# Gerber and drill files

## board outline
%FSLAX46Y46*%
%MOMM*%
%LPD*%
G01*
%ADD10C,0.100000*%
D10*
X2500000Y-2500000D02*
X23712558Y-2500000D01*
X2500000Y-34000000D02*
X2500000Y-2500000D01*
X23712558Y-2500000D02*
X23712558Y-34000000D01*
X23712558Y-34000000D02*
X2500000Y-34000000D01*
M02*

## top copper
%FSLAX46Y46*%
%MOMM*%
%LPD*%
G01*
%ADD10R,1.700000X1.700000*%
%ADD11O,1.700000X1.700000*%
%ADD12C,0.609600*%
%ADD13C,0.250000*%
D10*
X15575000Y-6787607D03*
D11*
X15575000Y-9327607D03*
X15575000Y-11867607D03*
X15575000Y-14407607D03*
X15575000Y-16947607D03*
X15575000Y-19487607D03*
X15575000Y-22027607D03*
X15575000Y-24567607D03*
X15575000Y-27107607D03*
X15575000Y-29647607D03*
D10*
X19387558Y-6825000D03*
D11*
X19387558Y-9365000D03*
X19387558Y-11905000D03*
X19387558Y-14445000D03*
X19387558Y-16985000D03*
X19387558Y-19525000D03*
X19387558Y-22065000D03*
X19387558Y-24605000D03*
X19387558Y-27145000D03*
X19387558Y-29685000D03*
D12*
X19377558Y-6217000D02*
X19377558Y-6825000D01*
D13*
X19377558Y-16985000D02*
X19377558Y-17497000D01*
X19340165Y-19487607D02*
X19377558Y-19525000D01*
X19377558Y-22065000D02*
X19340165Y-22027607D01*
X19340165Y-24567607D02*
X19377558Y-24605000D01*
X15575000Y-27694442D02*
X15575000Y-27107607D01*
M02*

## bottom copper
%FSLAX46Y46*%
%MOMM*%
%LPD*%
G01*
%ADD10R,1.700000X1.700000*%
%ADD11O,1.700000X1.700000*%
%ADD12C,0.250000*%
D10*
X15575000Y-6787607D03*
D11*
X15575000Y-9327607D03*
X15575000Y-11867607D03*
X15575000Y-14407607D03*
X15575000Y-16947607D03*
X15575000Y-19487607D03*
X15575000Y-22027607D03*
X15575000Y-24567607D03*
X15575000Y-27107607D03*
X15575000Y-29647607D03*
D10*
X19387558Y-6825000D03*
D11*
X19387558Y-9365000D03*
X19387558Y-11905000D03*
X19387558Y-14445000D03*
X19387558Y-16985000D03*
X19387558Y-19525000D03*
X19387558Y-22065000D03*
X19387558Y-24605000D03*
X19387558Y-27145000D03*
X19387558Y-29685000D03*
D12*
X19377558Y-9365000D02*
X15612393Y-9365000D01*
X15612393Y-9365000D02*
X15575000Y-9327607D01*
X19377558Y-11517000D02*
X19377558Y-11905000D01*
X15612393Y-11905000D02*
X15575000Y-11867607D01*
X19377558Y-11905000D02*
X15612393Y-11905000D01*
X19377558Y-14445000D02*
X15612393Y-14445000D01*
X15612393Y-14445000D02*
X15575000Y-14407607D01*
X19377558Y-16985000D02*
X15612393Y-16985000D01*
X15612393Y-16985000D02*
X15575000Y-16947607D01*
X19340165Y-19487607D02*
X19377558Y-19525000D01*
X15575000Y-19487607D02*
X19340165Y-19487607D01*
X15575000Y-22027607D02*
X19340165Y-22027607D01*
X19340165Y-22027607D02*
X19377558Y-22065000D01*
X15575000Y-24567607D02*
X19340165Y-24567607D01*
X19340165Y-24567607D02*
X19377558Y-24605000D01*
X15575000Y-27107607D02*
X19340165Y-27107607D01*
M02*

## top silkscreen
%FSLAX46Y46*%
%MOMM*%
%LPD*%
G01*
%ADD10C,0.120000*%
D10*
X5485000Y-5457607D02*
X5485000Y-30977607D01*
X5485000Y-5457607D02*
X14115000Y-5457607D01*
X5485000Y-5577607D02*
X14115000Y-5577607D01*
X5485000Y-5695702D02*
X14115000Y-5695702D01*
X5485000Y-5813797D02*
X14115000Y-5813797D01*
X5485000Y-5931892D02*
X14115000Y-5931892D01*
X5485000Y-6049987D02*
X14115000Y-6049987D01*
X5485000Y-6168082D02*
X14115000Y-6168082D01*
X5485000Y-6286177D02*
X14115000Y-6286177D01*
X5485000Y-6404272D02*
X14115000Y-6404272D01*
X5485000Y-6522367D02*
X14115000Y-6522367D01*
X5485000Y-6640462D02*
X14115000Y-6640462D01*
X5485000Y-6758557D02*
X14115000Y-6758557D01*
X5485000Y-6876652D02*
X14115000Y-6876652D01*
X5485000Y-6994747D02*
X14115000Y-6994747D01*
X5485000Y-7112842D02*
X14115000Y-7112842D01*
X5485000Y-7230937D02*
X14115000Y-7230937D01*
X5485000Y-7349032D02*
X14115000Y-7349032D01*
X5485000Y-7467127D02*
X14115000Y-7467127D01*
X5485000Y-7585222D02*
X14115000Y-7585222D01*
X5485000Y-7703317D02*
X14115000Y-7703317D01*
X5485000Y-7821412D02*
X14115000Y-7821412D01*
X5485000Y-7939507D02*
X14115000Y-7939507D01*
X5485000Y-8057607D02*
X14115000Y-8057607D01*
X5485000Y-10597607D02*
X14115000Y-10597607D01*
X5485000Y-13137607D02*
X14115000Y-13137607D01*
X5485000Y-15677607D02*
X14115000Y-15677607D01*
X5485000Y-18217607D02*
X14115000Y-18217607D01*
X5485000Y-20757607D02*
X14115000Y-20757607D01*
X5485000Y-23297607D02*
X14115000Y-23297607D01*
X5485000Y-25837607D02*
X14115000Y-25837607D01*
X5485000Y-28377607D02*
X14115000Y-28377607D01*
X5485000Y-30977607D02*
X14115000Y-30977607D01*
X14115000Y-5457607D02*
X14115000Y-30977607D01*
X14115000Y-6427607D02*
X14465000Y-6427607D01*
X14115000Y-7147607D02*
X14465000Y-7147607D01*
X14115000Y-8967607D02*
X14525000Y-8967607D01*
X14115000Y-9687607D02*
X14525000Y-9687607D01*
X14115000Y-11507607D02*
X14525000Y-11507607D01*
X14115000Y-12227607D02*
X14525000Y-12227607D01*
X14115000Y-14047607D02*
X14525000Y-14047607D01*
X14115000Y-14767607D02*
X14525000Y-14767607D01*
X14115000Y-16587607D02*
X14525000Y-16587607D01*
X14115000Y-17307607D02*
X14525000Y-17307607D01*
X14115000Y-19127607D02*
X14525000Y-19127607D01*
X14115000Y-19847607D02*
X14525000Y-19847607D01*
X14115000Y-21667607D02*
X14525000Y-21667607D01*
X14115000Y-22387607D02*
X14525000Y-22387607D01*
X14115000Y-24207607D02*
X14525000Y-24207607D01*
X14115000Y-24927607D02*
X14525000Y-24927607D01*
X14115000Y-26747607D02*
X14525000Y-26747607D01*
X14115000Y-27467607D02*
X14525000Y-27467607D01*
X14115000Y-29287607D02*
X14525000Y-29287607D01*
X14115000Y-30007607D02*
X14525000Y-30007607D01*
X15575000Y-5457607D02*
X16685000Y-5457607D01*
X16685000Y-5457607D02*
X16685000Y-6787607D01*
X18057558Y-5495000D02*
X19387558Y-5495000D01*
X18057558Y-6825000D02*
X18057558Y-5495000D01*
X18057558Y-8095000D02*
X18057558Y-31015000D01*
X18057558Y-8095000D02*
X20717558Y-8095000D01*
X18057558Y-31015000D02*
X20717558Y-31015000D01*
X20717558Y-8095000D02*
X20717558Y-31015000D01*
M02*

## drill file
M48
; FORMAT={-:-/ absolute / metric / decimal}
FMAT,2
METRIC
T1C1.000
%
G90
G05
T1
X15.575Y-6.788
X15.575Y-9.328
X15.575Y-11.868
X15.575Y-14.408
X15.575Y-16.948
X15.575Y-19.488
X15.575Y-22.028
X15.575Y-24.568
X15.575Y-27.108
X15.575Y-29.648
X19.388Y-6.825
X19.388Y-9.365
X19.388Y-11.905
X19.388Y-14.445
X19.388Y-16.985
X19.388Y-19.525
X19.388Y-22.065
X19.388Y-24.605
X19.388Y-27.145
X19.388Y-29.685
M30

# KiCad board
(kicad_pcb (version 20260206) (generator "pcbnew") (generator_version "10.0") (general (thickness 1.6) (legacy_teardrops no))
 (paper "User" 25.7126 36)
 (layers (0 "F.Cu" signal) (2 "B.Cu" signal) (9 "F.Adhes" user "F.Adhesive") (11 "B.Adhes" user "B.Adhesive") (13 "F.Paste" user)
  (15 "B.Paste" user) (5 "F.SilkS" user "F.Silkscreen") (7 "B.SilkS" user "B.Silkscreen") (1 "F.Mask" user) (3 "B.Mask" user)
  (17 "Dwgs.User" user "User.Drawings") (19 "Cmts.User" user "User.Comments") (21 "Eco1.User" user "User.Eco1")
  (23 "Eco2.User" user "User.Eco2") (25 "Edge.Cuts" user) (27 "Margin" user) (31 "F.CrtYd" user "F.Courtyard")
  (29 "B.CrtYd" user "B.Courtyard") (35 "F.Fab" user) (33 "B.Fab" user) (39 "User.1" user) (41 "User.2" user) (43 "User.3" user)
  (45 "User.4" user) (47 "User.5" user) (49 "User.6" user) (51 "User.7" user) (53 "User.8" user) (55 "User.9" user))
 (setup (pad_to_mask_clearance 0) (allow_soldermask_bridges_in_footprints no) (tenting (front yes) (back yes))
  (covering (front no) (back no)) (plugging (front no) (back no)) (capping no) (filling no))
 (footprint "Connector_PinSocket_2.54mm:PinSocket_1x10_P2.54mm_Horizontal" (layer "F.Cu") (at 15.575 6.787607)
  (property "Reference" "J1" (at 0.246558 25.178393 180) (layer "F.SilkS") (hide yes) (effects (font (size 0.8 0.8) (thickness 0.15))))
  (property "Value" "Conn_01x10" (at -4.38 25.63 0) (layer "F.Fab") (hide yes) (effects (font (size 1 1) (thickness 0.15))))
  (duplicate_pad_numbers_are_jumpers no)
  (fp_line (start -10.09 -1.33) (end -10.09 24.19) (stroke (width 0.12) (type solid)) (layer "F.SilkS"))
  (fp_line (start -10.09 -1.33) (end -1.46 -1.33) (stroke (width 0.12) (type solid)) (layer "F.SilkS"))
  (fp_line (start -10.09 -1.21) (end -1.46 -1.21) (stroke (width 0.12) (type solid)) (layer "F.SilkS"))
  (fp_line (start -10.09 -1.091905) (end -1.46 -1.091905) (stroke (width 0.12) (type solid)) (layer "F.SilkS"))
  (fp_line (start -10.09 -0.97381) (end -1.46 -0.97381) (stroke (width 0.12) (type solid)) (layer "F.SilkS"))
  (fp_line (start -10.09 -0.855715) (end -1.46 -0.855715) (stroke (width 0.12) (type solid)) (layer "F.SilkS"))
  (fp_line (start -10.09 -0.73762) (end -1.46 -0.73762) (stroke (width 0.12) (type solid)) (layer "F.SilkS"))
  (fp_line (start -10.09 -0.619525) (end -1.46 -0.619525) (stroke (width 0.12) (type solid)) (layer "F.SilkS"))
  (fp_line (start -10.09 -0.50143) (end -1.46 -0.50143) (stroke (width 0.12) (type solid)) (layer "F.SilkS"))
  (fp_line (start -10.09 -0.383335) (end -1.46 -0.383335) (stroke (width 0.12) (type solid)) (layer "F.SilkS"))
  (fp_line (start -10.09 -0.26524) (end -1.46 -0.26524) (stroke (width 0.12) (type solid)) (layer "F.SilkS"))
  (fp_line (start -10.09 -0.147145) (end -1.46 -0.147145) (stroke (width 0.12) (type solid)) (layer "F.SilkS"))
  (fp_line (start -10.09 -0.02905) (end -1.46 -0.02905) (stroke (width 0.12) (type solid)) (layer "F.SilkS"))
  (fp_line (start -10.09 0.089045) (end -1.46 0.089045) (stroke (width 0.12) (type solid)) (layer "F.SilkS"))
  (fp_line (start -10.09 0.20714) (end -1.46 0.20714) (stroke (width 0.12) (type solid)) (layer "F.SilkS"))
  (fp_line (start -10.09 0.325235) (end -1.46 0.325235) (stroke (width 0.12) (type solid)) (layer "F.SilkS"))
  (fp_line (start -10.09 0.44333) (end -1.46 0.44333) (stroke (width 0.12) (type solid)) (layer "F.SilkS"))
  (fp_line (start -10.09 0.561425) (end -1.46 0.561425) (stroke (width 0.12) (type solid)) (layer "F.SilkS"))
  (fp_line (start -10.09 0.67952) (end -1.46 0.67952) (stroke (width 0.12) (type solid)) (layer "F.SilkS"))
  (fp_line (start -10.09 0.797615) (end -1.46 0.797615) (stroke (width 0.12) (type solid)) (layer "F.SilkS"))
  (fp_line (start -10.09 0.91571) (end -1.46 0.91571) (stroke (width 0.12) (type solid)) (layer "F.SilkS"))
  (fp_line (start -10.09 1.033805) (end -1.46 1.033805) (stroke (width 0.12) (type solid)) (layer "F.SilkS"))
  (fp_line (start -10.09 1.1519) (end -1.46 1.1519) (stroke (width 0.12) (type solid)) (layer "F.SilkS"))
  (fp_line (start -10.09 1.27) (end -1.46 1.27) (stroke (width 0.12) (type solid)) (layer "F.SilkS"))
  (fp_line (start -10.09 3.81) (end -1.46 3.81) (stroke (width 0.12) (type solid)) (layer "F.SilkS"))
  (fp_line (start -10.09 6.35) (end -1.46 6.35) (stroke (width 0.12) (type solid)) (layer "F.SilkS"))
  (fp_line (start -10.09 8.89) (end -1.46 8.89) (stroke (width 0.12) (type solid)) (layer "F.SilkS"))
  (fp_line (start -10.09 11.43) (end -1.46 11.43) (stroke (width 0.12) (type solid)) (layer "F.SilkS"))
  (fp_line (start -10.09 13.97) (end -1.46 13.97) (stroke (width 0.12) (type solid)) (layer "F.SilkS"))
  (fp_line (start -10.09 16.51) (end -1.46 16.51) (stroke (width 0.12) (type solid)) (layer "F.SilkS"))
  (fp_line (start -10.09 19.05) (end -1.46 19.05) (stroke (width 0.12) (type solid)) (layer "F.SilkS"))
  (fp_line (start -10.09 21.59) (end -1.46 21.59) (stroke (width 0.12) (type solid)) (layer "F.SilkS"))
  (fp_line (start -10.09 24.19) (end -1.46 24.19) (stroke (width 0.12) (type solid)) (layer "F.SilkS"))
  (fp_line (start -1.46 -1.33) (end -1.46 24.19) (stroke (width 0.12) (type solid)) (layer "F.SilkS"))
  (fp_line (start -1.46 -0.36) (end -1.11 -0.36) (stroke (width 0.12) (type solid)) (layer "F.SilkS"))
  (fp_line (start -1.46 0.36) (end -1.11 0.36) (stroke (width 0.12) (type solid)) (layer "F.SilkS"))
  (fp_line (start -1.46 2.18) (end -1.05 2.18) (stroke (width 0.12) (type solid)) (layer "F.SilkS"))
  (fp_line (start -1.46 2.9) (end -1.05 2.9) (stroke (width 0.12) (type solid)) (layer "F.SilkS"))
  (fp_line (start -1.46 4.72) (end -1.05 4.72) (stroke (width 0.12) (type solid)) (layer "F.SilkS"))
  (fp_line (start -1.46 5.44) (end -1.05 5.44) (stroke (width 0.12) (type solid)) (layer "F.SilkS"))
  (fp_line (start -1.46 7.26) (end -1.05 7.26) (stroke (width 0.12) (type solid)) (layer "F.SilkS"))
  (fp_line (start -1.46 7.98) (end -1.05 7.98) (stroke (width 0.12) (type solid)) (layer "F.SilkS"))
  (fp_line (start -1.46 9.8) (end -1.05 9.8) (stroke (width 0.12) (type solid)) (layer "F.SilkS"))
  (fp_line (start -1.46 10.52) (end -1.05 10.52) (stroke (width 0.12) (type solid)) (layer "F.SilkS"))
  (fp_line (start -1.46 12.34) (end -1.05 12.34) (stroke (width 0.12) (type solid)) (layer "F.SilkS"))
  (fp_line (start -1.46 13.06) (end -1.05 13.06) (stroke (width 0.12) (type solid)) (layer "F.SilkS"))
  (fp_line (start -1.46 14.88) (end -1.05 14.88) (stroke (width 0.12) (type solid)) (layer "F.SilkS"))
  (fp_line (start -1.46 15.6) (end -1.05 15.6) (stroke (width 0.12) (type solid)) (layer "F.SilkS"))
  (fp_line (start -1.46 17.42) (end -1.05 17.42) (stroke (width 0.12) (type solid)) (layer "F.SilkS"))
  (fp_line (start -1.46 18.14) (end -1.05 18.14) (stroke (width 0.12) (type solid)) (layer "F.SilkS"))
  (fp_line (start -1.46 19.96) (end -1.05 19.96) (stroke (width 0.12) (type solid)) (layer "F.SilkS"))
  (fp_line (start -1.46 20.68) (end -1.05 20.68) (stroke (width 0.12) (type solid)) (layer "F.SilkS"))
  (fp_line (start -1.46 22.5) (end -1.05 22.5) (stroke (width 0.12) (type solid)) (layer "F.SilkS"))
  (fp_line (start -1.46 23.22) (end -1.05 23.22) (stroke (width 0.12) (type solid)) (layer "F.SilkS"))
  (fp_line (start 0 -1.33) (end 1.11 -1.33) (stroke (width 0.12) (type solid)) (layer "F.SilkS"))
  (fp_line (start 1.11 -1.33) (end 1.11 0) (stroke (width 0.12) (type solid)) (layer "F.SilkS"))
  (pad "1" thru_hole rect (at 0 0) (size 1.7 1.7) (drill 1) (layers "*.Cu" "*.Mask") (remove_unused_layers no) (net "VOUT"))
  (pad "2" thru_hole oval (at 0 2.54) (size 1.7 1.7) (drill 1) (layers "*.Cu" "*.Mask") (remove_unused_layers no) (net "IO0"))
  (pad "3" thru_hole oval (at 0 5.08) (size 1.7 1.7) (drill 1) (layers "*.Cu" "*.Mask") (remove_unused_layers no) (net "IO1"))
  (pad "4" thru_hole oval (at 0 7.62) (size 1.7 1.7) (drill 1) (layers "*.Cu" "*.Mask") (remove_unused_layers no) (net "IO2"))
  (pad "5" thru_hole oval (at 0 10.16) (size 1.7 1.7) (drill 1) (layers "*.Cu" "*.Mask") (remove_unused_layers no) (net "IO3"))
  (pad "6" thru_hole oval (at 0 12.7) (size 1.7 1.7) (drill 1) (layers "*.Cu" "*.Mask") (remove_unused_layers no) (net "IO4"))
  (pad "7" thru_hole oval (at 0 15.24) (size 1.7 1.7) (drill 1) (layers "*.Cu" "*.Mask") (remove_unused_layers no) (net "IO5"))
  (pad "8" thru_hole oval (at 0 17.78) (size 1.7 1.7) (drill 1) (layers "*.Cu" "*.Mask") (remove_unused_layers no) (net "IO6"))
  (pad "9" thru_hole oval (at 0 20.32) (size 1.7 1.7) (drill 1) (layers "*.Cu" "*.Mask") (remove_unused_layers no) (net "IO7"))
  (pad "10" thru_hole oval (at 0 22.86) (size 1.7 1.7) (drill 1) (layers "*.Cu" "*.Mask") (remove_unused_layers no) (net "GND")))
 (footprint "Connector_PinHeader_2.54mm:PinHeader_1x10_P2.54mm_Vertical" (layer "F.Cu") (at 19.387558 6.825)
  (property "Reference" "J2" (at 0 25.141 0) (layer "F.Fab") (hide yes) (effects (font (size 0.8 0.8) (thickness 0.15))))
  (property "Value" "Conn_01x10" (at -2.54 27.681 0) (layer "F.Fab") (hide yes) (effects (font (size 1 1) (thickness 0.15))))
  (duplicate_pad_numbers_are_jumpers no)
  (fp_line (start -1.33 -1.33) (end 0 -1.33) (stroke (width 0.12) (type solid)) (layer "F.SilkS"))
  (fp_line (start -1.33 0) (end -1.33 -1.33) (stroke (width 0.12) (type solid)) (layer "F.SilkS"))
  (fp_line (start -1.33 1.27) (end -1.33 24.19) (stroke (width 0.12) (type solid)) (layer "F.SilkS"))
  (fp_line (start -1.33 1.27) (end 1.33 1.27) (stroke (width 0.12) (type solid)) (layer "F.SilkS"))
  (fp_line (start -1.33 24.19) (end 1.33 24.19) (stroke (width 0.12) (type solid)) (layer "F.SilkS"))
  (fp_line (start 1.33 1.27) (end 1.33 24.19) (stroke (width 0.12) (type solid)) (layer "F.SilkS"))
  (pad "1" thru_hole rect (at 0 0) (size 1.7 1.7) (drill 1) (layers "*.Cu" "*.Mask") (remove_unused_layers no) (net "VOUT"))
  (pad "2" thru_hole oval (at 0 2.54) (size 1.7 1.7) (drill 1) (layers "*.Cu" "*.Mask") (remove_unused_layers no) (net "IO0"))
  (pad "3" thru_hole oval (at 0 5.08) (size 1.7 1.7) (drill 1) (layers "*.Cu" "*.Mask") (remove_unused_layers no) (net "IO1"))
  (pad "4" thru_hole oval (at 0 7.62) (size 1.7 1.7) (drill 1) (layers "*.Cu" "*.Mask") (remove_unused_layers no) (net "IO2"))
  (pad "5" thru_hole oval (at 0 10.16) (size 1.7 1.7) (drill 1) (layers "*.Cu" "*.Mask") (remove_unused_layers no) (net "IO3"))
  (pad "6" thru_hole oval (at 0 12.7) (size 1.7 1.7) (drill 1) (layers "*.Cu" "*.Mask") (remove_unused_layers no) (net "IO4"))
  (pad "7" thru_hole oval (at 0 15.24) (size 1.7 1.7) (drill 1) (layers "*.Cu" "*.Mask") (remove_unused_layers no) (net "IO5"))
  (pad "8" thru_hole oval (at 0 17.78) (size 1.7 1.7) (drill 1) (layers "*.Cu" "*.Mask") (remove_unused_layers no) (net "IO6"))
  (pad "9" thru_hole oval (at 0 20.32) (size 1.7 1.7) (drill 1) (layers "*.Cu" "*.Mask") (remove_unused_layers no) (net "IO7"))
  (pad "10" thru_hole oval (at 0 22.86) (size 1.7 1.7) (drill 1) (layers "*.Cu" "*.Mask") (remove_unused_layers no) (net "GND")))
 (gr_line (start 2.5 2.5) (end 23.712558 2.5) (stroke (width 0.1) (type default)) (layer "Edge.Cuts"))
 (gr_line (start 2.5 34) (end 2.5 2.5) (stroke (width 0.1) (type default)) (layer "Edge.Cuts"))
 (gr_line (start 23.712558 2.5) (end 23.712558 34) (stroke (width 0.1) (type default)) (layer "Edge.Cuts"))
 (gr_line (start 23.712558 34) (end 2.5 34) (stroke (width 0.1) (type default)) (layer "Edge.Cuts"))
 (segment (start 19.377558 6.217) (end 19.377558 6.825) (width 0.6096) (layer "F.Cu") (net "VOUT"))
 (segment (start 19.377558 9.365) (end 15.612393 9.365) (width 0.25) (layer "B.Cu") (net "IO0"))
 (segment (start 15.612393 9.365) (end 15.575 9.327607) (width 0.25) (layer "B.Cu") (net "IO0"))
 (segment (start 19.377558 11.517) (end 19.377558 11.905) (width 0.25) (layer "B.Cu") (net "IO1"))
 (segment (start 15.612393 11.905) (end 15.575 11.867607) (width 0.25) (layer "B.Cu") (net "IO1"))
 (segment (start 19.377558 11.905) (end 15.612393 11.905) (width 0.25) (layer "B.Cu") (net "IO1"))
 (segment (start 19.377558 14.445) (end 15.612393 14.445) (width 0.25) (layer "B.Cu") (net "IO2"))
 (segment (start 15.612393 14.445) (end 15.575 14.407607) (width 0.25) (layer "B.Cu") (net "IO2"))
 (segment (start 19.377558 16.985) (end 19.377558 17.497) (width 0.25) (layer "F.Cu") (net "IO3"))
 (segment (start 19.377558 16.985) (end 15.612393 16.985) (width 0.25) (layer "B.Cu") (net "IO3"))
 (segment (start 15.612393 16.985) (end 15.575 16.947607) (width 0.25) (layer "B.Cu") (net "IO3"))
 (segment (start 19.340165 19.487607) (end 19.377558 19.525) (width 0.25) (layer "F.Cu") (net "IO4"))
 (segment (start 19.340165 19.487607) (end 19.377558 19.525) (width 0.25) (layer "B.Cu") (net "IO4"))
 (segment (start 15.575 19.487607) (end 19.340165 19.487607) (width 0.25) (layer "B.Cu") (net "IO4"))
 (segment (start 19.377558 22.065) (end 19.340165 22.027607) (width 0.25) (layer "F.Cu") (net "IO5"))
 (segment (start 15.575 22.027607) (end 19.340165 22.027607) (width 0.25) (layer "B.Cu") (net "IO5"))
 (segment (start 19.340165 22.027607) (end 19.377558 22.065) (width 0.25) (layer "B.Cu") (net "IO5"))
 (segment (start 19.340165 24.567607) (end 19.377558 24.605) (width 0.25) (layer "F.Cu") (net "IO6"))
 (segment (start 15.575 24.567607) (end 19.340165 24.567607) (width 0.25) (layer "B.Cu") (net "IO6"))
 (segment (start 19.340165 24.567607) (end 19.377558 24.605) (width 0.25) (layer "B.Cu") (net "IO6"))
 (segment (start 15.575 27.694442) (end 15.575 27.107607) (width 0.25) (layer "F.Cu") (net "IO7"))
 (segment (start 15.575 27.107607) (end 19.340165 27.107607) (width 0.25) (layer "B.Cu") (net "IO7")))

